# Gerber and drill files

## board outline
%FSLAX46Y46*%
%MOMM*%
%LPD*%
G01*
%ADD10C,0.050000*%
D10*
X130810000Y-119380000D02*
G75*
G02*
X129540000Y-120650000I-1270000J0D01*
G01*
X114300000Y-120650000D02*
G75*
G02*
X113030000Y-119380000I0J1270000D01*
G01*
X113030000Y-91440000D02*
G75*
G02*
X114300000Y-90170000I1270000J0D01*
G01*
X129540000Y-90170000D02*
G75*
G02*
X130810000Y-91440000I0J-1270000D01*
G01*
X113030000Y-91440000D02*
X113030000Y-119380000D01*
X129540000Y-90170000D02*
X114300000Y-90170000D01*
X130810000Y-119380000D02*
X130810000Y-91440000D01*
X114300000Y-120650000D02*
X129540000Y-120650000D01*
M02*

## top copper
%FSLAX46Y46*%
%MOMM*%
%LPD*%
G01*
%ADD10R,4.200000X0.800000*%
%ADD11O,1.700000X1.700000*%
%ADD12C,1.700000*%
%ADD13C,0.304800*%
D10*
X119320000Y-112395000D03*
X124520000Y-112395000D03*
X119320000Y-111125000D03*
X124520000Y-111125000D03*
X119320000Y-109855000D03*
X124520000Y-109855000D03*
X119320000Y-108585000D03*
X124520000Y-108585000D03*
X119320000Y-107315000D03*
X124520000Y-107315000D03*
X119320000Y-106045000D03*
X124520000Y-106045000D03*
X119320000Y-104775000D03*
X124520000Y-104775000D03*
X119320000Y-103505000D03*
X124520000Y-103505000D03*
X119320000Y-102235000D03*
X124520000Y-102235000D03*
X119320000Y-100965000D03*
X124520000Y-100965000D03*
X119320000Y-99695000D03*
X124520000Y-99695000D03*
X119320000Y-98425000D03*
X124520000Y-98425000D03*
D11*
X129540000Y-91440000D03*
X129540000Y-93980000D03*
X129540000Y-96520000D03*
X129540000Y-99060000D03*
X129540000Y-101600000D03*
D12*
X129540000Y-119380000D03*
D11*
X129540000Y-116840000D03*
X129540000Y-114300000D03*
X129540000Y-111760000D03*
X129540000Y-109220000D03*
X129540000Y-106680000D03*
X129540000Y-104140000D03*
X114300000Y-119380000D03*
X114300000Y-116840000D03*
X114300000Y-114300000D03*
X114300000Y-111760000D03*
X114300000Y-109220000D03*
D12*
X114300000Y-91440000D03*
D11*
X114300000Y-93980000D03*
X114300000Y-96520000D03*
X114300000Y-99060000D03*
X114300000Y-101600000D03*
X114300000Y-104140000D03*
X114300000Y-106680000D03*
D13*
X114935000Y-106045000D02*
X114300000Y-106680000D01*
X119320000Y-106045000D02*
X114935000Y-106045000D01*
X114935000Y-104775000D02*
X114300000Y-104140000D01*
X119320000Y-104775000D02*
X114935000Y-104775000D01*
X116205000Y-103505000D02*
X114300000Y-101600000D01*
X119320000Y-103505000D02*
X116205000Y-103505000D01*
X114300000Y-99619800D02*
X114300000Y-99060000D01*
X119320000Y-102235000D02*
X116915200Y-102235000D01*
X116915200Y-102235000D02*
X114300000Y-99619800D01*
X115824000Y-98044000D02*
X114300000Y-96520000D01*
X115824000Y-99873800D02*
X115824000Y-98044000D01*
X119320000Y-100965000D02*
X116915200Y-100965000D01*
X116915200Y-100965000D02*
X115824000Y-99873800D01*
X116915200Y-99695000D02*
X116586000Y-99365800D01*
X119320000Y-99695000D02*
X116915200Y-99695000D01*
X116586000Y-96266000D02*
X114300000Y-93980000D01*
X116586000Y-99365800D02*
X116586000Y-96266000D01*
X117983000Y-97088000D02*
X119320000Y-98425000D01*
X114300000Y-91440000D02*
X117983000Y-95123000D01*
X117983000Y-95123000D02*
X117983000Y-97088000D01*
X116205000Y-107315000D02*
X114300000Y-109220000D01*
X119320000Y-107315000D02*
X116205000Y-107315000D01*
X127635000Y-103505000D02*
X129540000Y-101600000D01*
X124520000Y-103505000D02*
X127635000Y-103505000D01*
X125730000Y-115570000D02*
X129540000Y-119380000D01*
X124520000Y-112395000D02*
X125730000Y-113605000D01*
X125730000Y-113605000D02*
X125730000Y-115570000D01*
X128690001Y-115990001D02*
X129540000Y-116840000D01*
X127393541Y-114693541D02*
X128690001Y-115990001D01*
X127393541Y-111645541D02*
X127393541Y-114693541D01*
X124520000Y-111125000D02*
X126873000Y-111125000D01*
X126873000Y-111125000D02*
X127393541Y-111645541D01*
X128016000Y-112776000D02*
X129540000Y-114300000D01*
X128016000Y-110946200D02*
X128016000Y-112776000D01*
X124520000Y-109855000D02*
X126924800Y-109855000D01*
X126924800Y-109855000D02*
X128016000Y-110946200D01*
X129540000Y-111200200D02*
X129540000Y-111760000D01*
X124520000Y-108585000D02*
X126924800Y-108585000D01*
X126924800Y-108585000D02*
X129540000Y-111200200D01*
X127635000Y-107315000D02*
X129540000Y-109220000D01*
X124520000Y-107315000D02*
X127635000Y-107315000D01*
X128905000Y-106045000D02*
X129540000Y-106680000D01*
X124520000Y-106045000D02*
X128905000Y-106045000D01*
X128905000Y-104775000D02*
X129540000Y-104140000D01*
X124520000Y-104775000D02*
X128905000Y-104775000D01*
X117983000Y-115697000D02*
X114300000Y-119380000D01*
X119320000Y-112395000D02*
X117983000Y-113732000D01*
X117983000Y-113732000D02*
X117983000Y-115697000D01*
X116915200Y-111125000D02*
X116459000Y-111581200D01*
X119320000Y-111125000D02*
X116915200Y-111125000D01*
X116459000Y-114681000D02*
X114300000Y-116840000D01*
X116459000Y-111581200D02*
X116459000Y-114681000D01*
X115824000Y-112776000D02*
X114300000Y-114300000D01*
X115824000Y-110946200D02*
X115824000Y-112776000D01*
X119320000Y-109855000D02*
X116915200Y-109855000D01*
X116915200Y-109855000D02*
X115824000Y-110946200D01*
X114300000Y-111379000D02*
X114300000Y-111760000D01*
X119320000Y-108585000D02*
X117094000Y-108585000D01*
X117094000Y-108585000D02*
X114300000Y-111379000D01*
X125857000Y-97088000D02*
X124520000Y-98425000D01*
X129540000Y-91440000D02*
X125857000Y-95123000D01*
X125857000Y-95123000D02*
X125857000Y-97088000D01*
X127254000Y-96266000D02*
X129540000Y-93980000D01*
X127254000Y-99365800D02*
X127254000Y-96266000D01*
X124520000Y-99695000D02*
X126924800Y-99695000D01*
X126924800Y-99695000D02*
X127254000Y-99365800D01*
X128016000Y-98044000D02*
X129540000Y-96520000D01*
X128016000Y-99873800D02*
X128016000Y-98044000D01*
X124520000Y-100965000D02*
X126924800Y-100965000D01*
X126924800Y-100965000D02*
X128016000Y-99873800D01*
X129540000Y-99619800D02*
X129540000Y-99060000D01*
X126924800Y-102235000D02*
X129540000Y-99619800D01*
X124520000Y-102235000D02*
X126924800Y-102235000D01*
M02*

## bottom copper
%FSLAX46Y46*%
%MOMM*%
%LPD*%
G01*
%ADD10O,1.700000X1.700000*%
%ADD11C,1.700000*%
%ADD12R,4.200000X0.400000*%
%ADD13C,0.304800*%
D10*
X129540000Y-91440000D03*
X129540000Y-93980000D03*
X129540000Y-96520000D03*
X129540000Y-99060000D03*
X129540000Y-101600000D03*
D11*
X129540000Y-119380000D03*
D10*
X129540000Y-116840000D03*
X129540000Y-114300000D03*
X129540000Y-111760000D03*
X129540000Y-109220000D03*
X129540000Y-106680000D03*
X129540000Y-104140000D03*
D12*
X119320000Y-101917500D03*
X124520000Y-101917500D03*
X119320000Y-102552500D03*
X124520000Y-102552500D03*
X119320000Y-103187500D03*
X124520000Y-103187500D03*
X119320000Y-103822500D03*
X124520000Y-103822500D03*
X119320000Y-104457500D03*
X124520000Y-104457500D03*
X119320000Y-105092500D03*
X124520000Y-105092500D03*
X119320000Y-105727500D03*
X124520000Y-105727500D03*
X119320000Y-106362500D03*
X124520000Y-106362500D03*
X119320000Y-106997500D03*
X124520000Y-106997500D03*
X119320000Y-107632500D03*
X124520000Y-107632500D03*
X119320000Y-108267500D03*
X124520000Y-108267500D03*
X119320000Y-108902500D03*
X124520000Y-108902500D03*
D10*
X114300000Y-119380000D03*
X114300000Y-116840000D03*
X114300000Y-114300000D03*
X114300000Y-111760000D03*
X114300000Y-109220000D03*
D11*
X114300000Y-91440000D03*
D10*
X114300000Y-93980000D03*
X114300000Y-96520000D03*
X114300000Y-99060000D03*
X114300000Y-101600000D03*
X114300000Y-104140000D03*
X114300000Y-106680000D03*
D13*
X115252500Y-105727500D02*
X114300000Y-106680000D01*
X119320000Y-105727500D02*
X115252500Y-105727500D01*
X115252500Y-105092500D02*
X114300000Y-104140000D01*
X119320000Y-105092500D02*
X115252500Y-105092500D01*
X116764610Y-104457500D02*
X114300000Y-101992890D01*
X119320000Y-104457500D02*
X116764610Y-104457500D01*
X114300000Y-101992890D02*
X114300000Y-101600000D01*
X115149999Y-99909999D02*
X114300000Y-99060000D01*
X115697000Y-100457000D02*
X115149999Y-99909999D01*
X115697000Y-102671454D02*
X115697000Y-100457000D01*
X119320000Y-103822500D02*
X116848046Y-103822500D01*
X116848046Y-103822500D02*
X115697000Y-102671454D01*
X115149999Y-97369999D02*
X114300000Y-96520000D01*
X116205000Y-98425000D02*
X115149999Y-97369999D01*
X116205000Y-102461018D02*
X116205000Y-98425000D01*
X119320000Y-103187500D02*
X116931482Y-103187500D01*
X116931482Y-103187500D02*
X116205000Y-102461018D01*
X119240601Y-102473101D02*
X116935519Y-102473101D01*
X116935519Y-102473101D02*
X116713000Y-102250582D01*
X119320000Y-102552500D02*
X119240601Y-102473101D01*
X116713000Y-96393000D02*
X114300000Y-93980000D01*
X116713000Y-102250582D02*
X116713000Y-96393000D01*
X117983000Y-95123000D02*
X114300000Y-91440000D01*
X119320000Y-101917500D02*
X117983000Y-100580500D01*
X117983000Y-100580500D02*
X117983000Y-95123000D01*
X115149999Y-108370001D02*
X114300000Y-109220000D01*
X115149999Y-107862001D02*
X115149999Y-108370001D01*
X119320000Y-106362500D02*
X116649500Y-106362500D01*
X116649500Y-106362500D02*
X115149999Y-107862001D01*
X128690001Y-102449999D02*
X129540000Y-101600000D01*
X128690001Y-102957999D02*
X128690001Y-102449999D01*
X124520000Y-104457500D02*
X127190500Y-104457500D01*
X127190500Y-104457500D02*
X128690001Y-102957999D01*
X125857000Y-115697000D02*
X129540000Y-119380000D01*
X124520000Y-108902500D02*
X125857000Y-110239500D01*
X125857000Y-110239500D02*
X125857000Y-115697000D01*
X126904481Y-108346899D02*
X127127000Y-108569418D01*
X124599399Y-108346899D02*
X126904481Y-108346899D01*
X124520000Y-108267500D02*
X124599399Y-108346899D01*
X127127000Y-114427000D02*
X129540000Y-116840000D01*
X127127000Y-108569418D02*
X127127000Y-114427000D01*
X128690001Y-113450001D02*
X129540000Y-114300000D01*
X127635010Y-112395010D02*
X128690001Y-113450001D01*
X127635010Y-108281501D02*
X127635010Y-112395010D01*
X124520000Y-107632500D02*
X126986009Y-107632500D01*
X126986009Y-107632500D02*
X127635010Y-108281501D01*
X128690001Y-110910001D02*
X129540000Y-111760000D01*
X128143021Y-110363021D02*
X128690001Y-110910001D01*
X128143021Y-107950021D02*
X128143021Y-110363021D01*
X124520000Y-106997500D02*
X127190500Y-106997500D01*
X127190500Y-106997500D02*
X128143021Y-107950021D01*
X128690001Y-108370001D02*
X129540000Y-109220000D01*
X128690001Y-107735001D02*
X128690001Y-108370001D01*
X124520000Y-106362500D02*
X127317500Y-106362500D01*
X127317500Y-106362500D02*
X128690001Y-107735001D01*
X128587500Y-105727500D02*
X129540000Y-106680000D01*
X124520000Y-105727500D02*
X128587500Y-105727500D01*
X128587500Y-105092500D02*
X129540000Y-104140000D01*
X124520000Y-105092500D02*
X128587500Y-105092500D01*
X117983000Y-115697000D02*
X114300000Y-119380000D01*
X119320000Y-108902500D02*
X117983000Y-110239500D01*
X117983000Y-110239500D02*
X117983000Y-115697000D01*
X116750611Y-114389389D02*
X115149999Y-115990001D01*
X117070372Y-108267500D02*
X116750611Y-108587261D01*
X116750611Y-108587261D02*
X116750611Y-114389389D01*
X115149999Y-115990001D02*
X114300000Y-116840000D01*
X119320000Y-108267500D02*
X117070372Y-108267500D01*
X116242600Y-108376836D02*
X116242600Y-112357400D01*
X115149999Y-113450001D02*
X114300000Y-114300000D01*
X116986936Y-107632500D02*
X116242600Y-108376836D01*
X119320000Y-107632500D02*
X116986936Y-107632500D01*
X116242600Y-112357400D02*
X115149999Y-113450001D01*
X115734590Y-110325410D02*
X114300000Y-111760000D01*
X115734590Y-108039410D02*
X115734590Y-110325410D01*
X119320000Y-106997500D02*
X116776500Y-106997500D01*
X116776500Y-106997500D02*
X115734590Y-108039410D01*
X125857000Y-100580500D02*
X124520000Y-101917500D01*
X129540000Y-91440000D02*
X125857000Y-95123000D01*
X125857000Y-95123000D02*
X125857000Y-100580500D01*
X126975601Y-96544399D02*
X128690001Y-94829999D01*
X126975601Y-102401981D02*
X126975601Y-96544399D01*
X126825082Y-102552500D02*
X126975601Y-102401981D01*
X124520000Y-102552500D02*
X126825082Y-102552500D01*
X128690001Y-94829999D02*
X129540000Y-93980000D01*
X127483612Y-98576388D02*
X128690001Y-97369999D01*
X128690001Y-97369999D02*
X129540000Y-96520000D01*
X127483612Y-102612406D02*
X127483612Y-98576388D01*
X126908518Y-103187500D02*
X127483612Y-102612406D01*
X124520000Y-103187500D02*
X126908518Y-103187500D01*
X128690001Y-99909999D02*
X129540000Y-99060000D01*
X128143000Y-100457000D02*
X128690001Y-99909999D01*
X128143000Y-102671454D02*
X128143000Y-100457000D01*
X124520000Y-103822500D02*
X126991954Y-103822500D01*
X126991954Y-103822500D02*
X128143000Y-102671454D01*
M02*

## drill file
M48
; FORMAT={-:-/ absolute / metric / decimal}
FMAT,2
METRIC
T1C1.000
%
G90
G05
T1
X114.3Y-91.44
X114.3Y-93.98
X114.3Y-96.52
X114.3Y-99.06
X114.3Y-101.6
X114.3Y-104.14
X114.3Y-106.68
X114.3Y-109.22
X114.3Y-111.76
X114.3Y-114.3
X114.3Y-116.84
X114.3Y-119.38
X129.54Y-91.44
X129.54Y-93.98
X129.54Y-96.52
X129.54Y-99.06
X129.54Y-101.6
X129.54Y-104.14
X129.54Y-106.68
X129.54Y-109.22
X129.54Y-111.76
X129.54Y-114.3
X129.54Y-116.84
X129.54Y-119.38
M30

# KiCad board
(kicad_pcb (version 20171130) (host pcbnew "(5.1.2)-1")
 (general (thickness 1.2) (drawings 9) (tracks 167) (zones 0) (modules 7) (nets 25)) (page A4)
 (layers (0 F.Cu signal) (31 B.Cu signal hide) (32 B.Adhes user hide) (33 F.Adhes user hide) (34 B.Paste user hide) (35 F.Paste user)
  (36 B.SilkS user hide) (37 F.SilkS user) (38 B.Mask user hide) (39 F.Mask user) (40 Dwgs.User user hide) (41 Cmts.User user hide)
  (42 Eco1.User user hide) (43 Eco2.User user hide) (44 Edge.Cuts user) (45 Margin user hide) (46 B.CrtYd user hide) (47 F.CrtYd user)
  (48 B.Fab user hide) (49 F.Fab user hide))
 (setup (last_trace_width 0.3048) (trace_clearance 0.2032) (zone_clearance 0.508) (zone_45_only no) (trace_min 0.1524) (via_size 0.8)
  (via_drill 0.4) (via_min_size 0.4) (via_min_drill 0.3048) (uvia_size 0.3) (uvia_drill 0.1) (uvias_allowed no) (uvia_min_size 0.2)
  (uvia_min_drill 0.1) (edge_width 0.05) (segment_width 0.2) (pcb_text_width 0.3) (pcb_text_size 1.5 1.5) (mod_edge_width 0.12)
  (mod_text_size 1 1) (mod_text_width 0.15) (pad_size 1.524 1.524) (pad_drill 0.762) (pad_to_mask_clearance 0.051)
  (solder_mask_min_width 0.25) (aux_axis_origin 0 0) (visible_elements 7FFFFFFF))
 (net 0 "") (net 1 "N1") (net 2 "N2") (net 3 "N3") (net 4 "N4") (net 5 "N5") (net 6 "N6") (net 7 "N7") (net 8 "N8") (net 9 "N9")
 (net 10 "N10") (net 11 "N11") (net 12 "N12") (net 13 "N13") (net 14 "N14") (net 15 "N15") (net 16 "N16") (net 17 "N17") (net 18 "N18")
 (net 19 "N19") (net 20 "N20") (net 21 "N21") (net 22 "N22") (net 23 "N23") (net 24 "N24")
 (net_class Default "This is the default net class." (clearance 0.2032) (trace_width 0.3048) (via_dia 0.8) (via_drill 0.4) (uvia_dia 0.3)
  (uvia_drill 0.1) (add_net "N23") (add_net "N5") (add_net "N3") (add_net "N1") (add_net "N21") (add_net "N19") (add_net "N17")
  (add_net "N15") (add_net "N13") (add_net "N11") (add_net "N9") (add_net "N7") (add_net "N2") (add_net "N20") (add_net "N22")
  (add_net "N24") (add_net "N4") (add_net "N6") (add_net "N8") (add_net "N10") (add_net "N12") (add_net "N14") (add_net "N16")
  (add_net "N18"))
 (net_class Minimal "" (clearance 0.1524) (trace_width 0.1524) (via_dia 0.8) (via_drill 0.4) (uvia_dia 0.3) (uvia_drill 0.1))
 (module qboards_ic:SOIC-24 (layer F.Cu) (at 121.92 105.41 270)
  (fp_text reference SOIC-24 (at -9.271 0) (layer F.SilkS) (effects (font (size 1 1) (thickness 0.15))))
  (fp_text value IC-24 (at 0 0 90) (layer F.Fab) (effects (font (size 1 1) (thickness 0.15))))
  (pad 12 smd rect (at 6.985 2.6 270) (size 0.8 4.2) (layers F.Cu F.Paste F.Mask) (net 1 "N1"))
  (pad 13 smd rect (at 6.985 -2.6 270) (size 0.8 4.2) (layers F.Cu F.Paste F.Mask) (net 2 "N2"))
  (pad 11 smd rect (at 5.715 2.6 270) (size 0.8 4.2) (layers F.Cu F.Paste F.Mask) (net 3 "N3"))
  (pad 14 smd rect (at 5.715 -2.6 270) (size 0.8 4.2) (layers F.Cu F.Paste F.Mask) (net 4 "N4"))
  (pad 10 smd rect (at 4.445 2.6 270) (size 0.8 4.2) (layers F.Cu F.Paste F.Mask) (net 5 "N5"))
  (pad 15 smd rect (at 4.445 -2.6 270) (size 0.8 4.2) (layers F.Cu F.Paste F.Mask) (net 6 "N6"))
  (pad 9 smd rect (at 3.175 2.6 270) (size 0.8 4.2) (layers F.Cu F.Paste F.Mask) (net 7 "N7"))
  (pad 16 smd rect (at 3.175 -2.6 270) (size 0.8 4.2) (layers F.Cu F.Paste F.Mask) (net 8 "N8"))
  (pad 8 smd rect (at 1.905 2.6 270) (size 0.8 4.2) (layers F.Cu F.Paste F.Mask) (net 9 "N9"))
  (pad 17 smd rect (at 1.905 -2.6 270) (size 0.8 4.2) (layers F.Cu F.Paste F.Mask) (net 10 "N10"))
  (pad 7 smd rect (at 0.635 2.6 270) (size 0.8 4.2) (layers F.Cu F.Paste F.Mask) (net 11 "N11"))
  (pad 18 smd rect (at 0.635 -2.6 270) (size 0.8 4.2) (layers F.Cu F.Paste F.Mask) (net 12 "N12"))
  (pad 6 smd rect (at -0.635 2.6 270) (size 0.8 4.2) (layers F.Cu F.Paste F.Mask) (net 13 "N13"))
  (pad 19 smd rect (at -0.635 -2.6 270) (size 0.8 4.2) (layers F.Cu F.Paste F.Mask) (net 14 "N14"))
  (pad 5 smd rect (at -1.905 2.6 270) (size 0.8 4.2) (layers F.Cu F.Paste F.Mask) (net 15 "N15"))
  (pad 20 smd rect (at -1.905 -2.6 270) (size 0.8 4.2) (layers F.Cu F.Paste F.Mask) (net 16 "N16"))
  (pad 4 smd rect (at -3.175 2.6 270) (size 0.8 4.2) (layers F.Cu F.Paste F.Mask) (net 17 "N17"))
  (pad 21 smd rect (at -3.175 -2.6 270) (size 0.8 4.2) (layers F.Cu F.Paste F.Mask) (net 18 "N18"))
  (pad 3 smd rect (at -4.445 2.6 270) (size 0.8 4.2) (layers F.Cu F.Paste F.Mask) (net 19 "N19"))
  (pad 22 smd rect (at -4.445 -2.6 270) (size 0.8 4.2) (layers F.Cu F.Paste F.Mask) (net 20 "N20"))
  (pad 2 smd rect (at -5.715 2.6 270) (size 0.8 4.2) (layers F.Cu F.Paste F.Mask) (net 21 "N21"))
  (pad 23 smd rect (at -5.715 -2.6 270) (size 0.8 4.2) (layers F.Cu F.Paste F.Mask) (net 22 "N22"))
  (pad 1 smd rect (at -6.985 2.6 270) (size 0.8 4.2) (layers F.Cu F.Paste F.Mask) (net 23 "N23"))
  (pad 24 smd rect (at -6.985 -2.6 270) (size 0.8 4.2) (layers F.Cu F.Paste F.Mask) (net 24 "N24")))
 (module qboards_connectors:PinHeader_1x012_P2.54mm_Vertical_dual (layer F.Cu) (at 129.54 119.38 180)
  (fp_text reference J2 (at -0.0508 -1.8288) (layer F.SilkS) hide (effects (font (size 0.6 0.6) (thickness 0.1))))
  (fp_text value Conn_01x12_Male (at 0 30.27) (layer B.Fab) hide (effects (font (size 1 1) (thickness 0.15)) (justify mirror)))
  (pad 12 thru_hole oval (at 0 27.94 180) (size 1.7 1.7) (drill 1) (layers *.Cu *.Mask) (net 24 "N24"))
  (pad 11 thru_hole oval (at 0 25.4 180) (size 1.7 1.7) (drill 1) (layers *.Cu *.Mask) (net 22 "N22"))
  (pad 10 thru_hole oval (at 0 22.86 180) (size 1.7 1.7) (drill 1) (layers *.Cu *.Mask) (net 20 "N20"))
  (pad 9 thru_hole oval (at 0 20.32 180) (size 1.7 1.7) (drill 1) (layers *.Cu *.Mask) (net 18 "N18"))
  (pad 8 thru_hole oval (at 0 17.78 180) (size 1.7 1.7) (drill 1) (layers *.Cu *.Mask) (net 16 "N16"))
  (pad 1 thru_hole circle (at 0 0 180) (size 1.7 1.7) (drill 1) (layers *.Cu *.Mask) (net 2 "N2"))
  (pad 2 thru_hole oval (at 0 2.54 180) (size 1.7 1.7) (drill 1) (layers *.Cu *.Mask) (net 4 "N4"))
  (pad 3 thru_hole oval (at 0 5.08 180) (size 1.7 1.7) (drill 1) (layers *.Cu *.Mask) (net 6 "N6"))
  (pad 4 thru_hole oval (at 0 7.62 180) (size 1.7 1.7) (drill 1) (layers *.Cu *.Mask) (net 8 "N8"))
  (pad 5 thru_hole oval (at 0 10.16 180) (size 1.7 1.7) (drill 1) (layers *.Cu *.Mask) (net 10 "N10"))
  (pad 6 thru_hole oval (at 0 12.7 180) (size 1.7 1.7) (drill 1) (layers *.Cu *.Mask) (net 12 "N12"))
  (pad 7 thru_hole oval (at 0 15.24 180) (size 1.7 1.7) (drill 1) (layers *.Cu *.Mask) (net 14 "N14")))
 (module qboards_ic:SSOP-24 (layer B.Cu) (at 121.92 105.41 90)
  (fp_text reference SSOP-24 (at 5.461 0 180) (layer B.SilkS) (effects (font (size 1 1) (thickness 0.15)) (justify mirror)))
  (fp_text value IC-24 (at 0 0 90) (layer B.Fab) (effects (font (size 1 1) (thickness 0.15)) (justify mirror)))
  (pad 12 smd rect (at 3.4925 -2.6 90) (size 0.4 4.2) (layers B.Cu B.Paste B.Mask) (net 23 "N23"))
  (pad 13 smd rect (at 3.4925 2.6 90) (size 0.4 4.2) (layers B.Cu B.Paste B.Mask) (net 24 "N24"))
  (pad 11 smd rect (at 2.8575 -2.6 90) (size 0.4 4.2) (layers B.Cu B.Paste B.Mask) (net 21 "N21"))
  (pad 14 smd rect (at 2.8575 2.6 90) (size 0.4 4.2) (layers B.Cu B.Paste B.Mask) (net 22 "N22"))
  (pad 10 smd rect (at 2.2225 -2.6 90) (size 0.4 4.2) (layers B.Cu B.Paste B.Mask) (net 19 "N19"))
  (pad 15 smd rect (at 2.2225 2.6 90) (size 0.4 4.2) (layers B.Cu B.Paste B.Mask) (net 20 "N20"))
  (pad 9 smd rect (at 1.5875 -2.6 90) (size 0.4 4.2) (layers B.Cu B.Paste B.Mask) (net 17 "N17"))
  (pad 16 smd rect (at 1.5875 2.6 90) (size 0.4 4.2) (layers B.Cu B.Paste B.Mask) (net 18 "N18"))
  (pad 8 smd rect (at 0.9525 -2.6 90) (size 0.4 4.2) (layers B.Cu B.Paste B.Mask) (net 15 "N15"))
  (pad 17 smd rect (at 0.9525 2.6 90) (size 0.4 4.2) (layers B.Cu B.Paste B.Mask) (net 16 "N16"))
  (pad 7 smd rect (at 0.3175 -2.6 90) (size 0.4 4.2) (layers B.Cu B.Paste B.Mask) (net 13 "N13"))
  (pad 18 smd rect (at 0.3175 2.6 90) (size 0.4 4.2) (layers B.Cu B.Paste B.Mask) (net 14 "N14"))
  (pad 6 smd rect (at -0.3175 -2.6 90) (size 0.4 4.2) (layers B.Cu B.Paste B.Mask) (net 11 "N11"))
  (pad 19 smd rect (at -0.3175 2.6 90) (size 0.4 4.2) (layers B.Cu B.Paste B.Mask) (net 12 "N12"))
  (pad 5 smd rect (at -0.9525 -2.6 90) (size 0.4 4.2) (layers B.Cu B.Paste B.Mask) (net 9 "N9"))
  (pad 20 smd rect (at -0.9525 2.6 90) (size 0.4 4.2) (layers B.Cu B.Paste B.Mask) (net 10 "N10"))
  (pad 4 smd rect (at -1.5875 -2.6 90) (size 0.4 4.2) (layers B.Cu B.Paste B.Mask) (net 7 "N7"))
  (pad 21 smd rect (at -1.5875 2.6 90) (size 0.4 4.2) (layers B.Cu B.Paste B.Mask) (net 8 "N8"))
  (pad 3 smd rect (at -2.2225 -2.6 90) (size 0.4 4.2) (layers B.Cu B.Paste B.Mask) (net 5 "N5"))
  (pad 22 smd rect (at -2.2225 2.6 90) (size 0.4 4.2) (layers B.Cu B.Paste B.Mask) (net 6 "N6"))
  (pad 2 smd rect (at -2.8575 -2.6 90) (size 0.4 4.2) (layers B.Cu B.Paste B.Mask) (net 3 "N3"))
  (pad 23 smd rect (at -2.8575 2.6 90) (size 0.4 4.2) (layers B.Cu B.Paste B.Mask) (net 4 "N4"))
  (pad 1 smd rect (at -3.4925 -2.6 90) (size 0.4 4.2) (layers B.Cu B.Paste B.Mask) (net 1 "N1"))
  (pad 24 smd rect (at -3.4925 2.6 90) (size 0.4 4.2) (layers B.Cu B.Paste B.Mask) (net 2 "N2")))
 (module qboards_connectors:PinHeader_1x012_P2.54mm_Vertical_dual (layer F.Cu) (at 114.3 91.44)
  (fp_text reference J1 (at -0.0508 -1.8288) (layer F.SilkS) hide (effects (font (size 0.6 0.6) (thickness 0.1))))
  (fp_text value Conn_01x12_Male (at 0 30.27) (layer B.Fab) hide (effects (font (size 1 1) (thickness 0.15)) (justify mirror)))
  (pad 12 thru_hole oval (at 0 27.94) (size 1.7 1.7) (drill 1) (layers *.Cu *.Mask) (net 1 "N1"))
  (pad 11 thru_hole oval (at 0 25.4) (size 1.7 1.7) (drill 1) (layers *.Cu *.Mask) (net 3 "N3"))
  (pad 10 thru_hole oval (at 0 22.86) (size 1.7 1.7) (drill 1) (layers *.Cu *.Mask) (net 5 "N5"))
  (pad 9 thru_hole oval (at 0 20.32) (size 1.7 1.7) (drill 1) (layers *.Cu *.Mask) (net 7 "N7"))
  (pad 8 thru_hole oval (at 0 17.78) (size 1.7 1.7) (drill 1) (layers *.Cu *.Mask) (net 9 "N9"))
  (pad 1 thru_hole circle (at 0 0) (size 1.7 1.7) (drill 1) (layers *.Cu *.Mask) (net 23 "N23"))
  (pad 2 thru_hole oval (at 0 2.54) (size 1.7 1.7) (drill 1) (layers *.Cu *.Mask) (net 21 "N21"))
  (pad 3 thru_hole oval (at 0 5.08) (size 1.7 1.7) (drill 1) (layers *.Cu *.Mask) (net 19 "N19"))
  (pad 4 thru_hole oval (at 0 7.62) (size 1.7 1.7) (drill 1) (layers *.Cu *.Mask) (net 17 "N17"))
  (pad 5 thru_hole oval (at 0 10.16) (size 1.7 1.7) (drill 1) (layers *.Cu *.Mask) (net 15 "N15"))
  (pad 6 thru_hole oval (at 0 12.7) (size 1.7 1.7) (drill 1) (layers *.Cu *.Mask) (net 13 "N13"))
  (pad 7 thru_hole oval (at 0 15.24) (size 1.7 1.7) (drill 1) (layers *.Cu *.Mask) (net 11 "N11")))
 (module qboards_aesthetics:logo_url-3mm (layer F.Cu) (at 117.602 117.983)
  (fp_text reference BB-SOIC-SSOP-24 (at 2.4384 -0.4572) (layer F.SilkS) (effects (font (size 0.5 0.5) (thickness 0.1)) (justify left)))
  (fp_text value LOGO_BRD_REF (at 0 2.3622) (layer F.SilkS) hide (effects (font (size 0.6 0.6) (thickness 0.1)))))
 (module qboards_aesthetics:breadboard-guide (layer F.Cu) (at 99.06 91.44)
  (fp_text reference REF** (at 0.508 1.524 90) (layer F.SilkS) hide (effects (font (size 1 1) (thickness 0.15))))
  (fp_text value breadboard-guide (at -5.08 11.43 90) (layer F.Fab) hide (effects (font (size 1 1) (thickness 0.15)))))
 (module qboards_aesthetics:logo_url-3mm (layer B.Cu) (at 126.492 117.983 180)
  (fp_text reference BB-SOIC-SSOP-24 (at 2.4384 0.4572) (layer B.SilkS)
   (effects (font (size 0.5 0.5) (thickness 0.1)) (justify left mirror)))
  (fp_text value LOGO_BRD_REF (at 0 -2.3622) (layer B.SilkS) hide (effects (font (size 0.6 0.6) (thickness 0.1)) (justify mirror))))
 (gr_arc (start 129.54 119.38) (end 129.54 120.65) (angle -90) (layer Edge.Cuts) (width 0.05))
 (gr_arc (start 114.3 119.38) (end 113.03 119.38) (angle -90) (layer Edge.Cuts) (width 0.05))
 (gr_arc (start 114.3 91.44) (end 114.3 90.17) (angle -90) (layer Edge.Cuts) (width 0.05))
 (gr_arc (start 129.54 91.44) (end 130.81 91.44) (angle -90) (layer Edge.Cuts) (width 0.05))
 (gr_line (start 113.03 91.44) (end 113.03 119.38) (layer Edge.Cuts) (width 0.05))
 (gr_line (start 129.54 90.17) (end 114.3 90.17) (layer Edge.Cuts) (width 0.05))
 (gr_line (start 130.81 119.38) (end 130.81 91.44) (layer Edge.Cuts) (width 0.05))
 (gr_line (start 114.3 120.65) (end 129.54 120.65) (layer Edge.Cuts) (width 0.05))
 (segment (start 114.935 106.045) (end 114.3 106.68) (width 0.3048) (layer F.Cu) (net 11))
 (segment (start 119.32 106.045) (end 114.935 106.045) (width 0.3048) (layer F.Cu) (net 11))
 (segment (start 115.2525 105.7275) (end 114.3 106.68) (width 0.3048) (layer B.Cu) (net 11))
 (segment (start 119.32 105.7275) (end 115.2525 105.7275) (width 0.3048) (layer B.Cu) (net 11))
 (segment (start 114.935 104.775) (end 114.3 104.14) (width 0.3048) (layer F.Cu) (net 13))
 (segment (start 119.32 104.775) (end 114.935 104.775) (width 0.3048) (layer F.Cu) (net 13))
 (segment (start 115.2525 105.0925) (end 114.3 104.14) (width 0.3048) (layer B.Cu) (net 13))
 (segment (start 119.32 105.0925) (end 115.2525 105.0925) (width 0.3048) (layer B.Cu) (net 13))
 (segment (start 116.205 103.505) (end 114.3 101.6) (width 0.3048) (layer F.Cu) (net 15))
 (segment (start 119.32 103.505) (end 116.205 103.505) (width 0.3048) (layer F.Cu) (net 15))
 (segment (start 116.76461 104.4575) (end 114.3 101.99289) (width 0.3048) (layer B.Cu) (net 15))
 (segment (start 119.32 104.4575) (end 116.76461 104.4575) (width 0.3048) (layer B.Cu) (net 15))
 (segment (start 114.3 101.99289) (end 114.3 101.6) (width 0.3048) (layer B.Cu) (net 15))
 (segment (start 114.3 99.6198) (end 114.3 99.06) (width 0.3048) (layer F.Cu) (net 17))
 (segment (start 119.32 102.235) (end 116.9152 102.235) (width 0.3048) (layer F.Cu) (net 17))
 (segment (start 116.9152 102.235) (end 114.3 99.6198) (width 0.3048) (layer F.Cu) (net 17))
 (segment (start 115.149999 99.909999) (end 114.3 99.06) (width 0.3048) (layer B.Cu) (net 17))
 (segment (start 115.697 100.457) (end 115.149999 99.909999) (width 0.3048) (layer B.Cu) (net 17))
 (segment (start 115.697 102.671454) (end 115.697 100.457) (width 0.3048) (layer B.Cu) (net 17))
 (segment (start 119.32 103.8225) (end 116.848046 103.8225) (width 0.3048) (layer B.Cu) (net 17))
 (segment (start 116.848046 103.8225) (end 115.697 102.671454) (width 0.3048) (layer B.Cu) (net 17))
 (segment (start 115.824 98.044) (end 114.3 96.52) (width 0.3048) (layer F.Cu) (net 19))
 (segment (start 115.824 99.8738) (end 115.824 98.044) (width 0.3048) (layer F.Cu) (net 19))
 (segment (start 119.32 100.965) (end 116.9152 100.965) (width 0.3048) (layer F.Cu) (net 19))
 (segment (start 116.9152 100.965) (end 115.824 99.8738) (width 0.3048) (layer F.Cu) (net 19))
 (segment (start 115.149999 97.369999) (end 114.3 96.52) (width 0.3048) (layer B.Cu) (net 19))
 (segment (start 116.205 98.425) (end 115.149999 97.369999) (width 0.3048) (layer B.Cu) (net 19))
 (segment (start 116.205 102.461018) (end 116.205 98.425) (width 0.3048) (layer B.Cu) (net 19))
 (segment (start 119.32 103.1875) (end 116.931482 103.1875) (width 0.3048) (layer B.Cu) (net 19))
 (segment (start 116.931482 103.1875) (end 116.205 102.461018) (width 0.3048) (layer B.Cu) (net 19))
 (segment (start 116.9152 99.695) (end 116.586 99.3658) (width 0.3048) (layer F.Cu) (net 21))
 (segment (start 119.32 99.695) (end 116.9152 99.695) (width 0.3048) (layer F.Cu) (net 21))
 (segment (start 116.586 96.266) (end 114.3 93.98) (width 0.3048) (layer F.Cu) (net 21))
 (segment (start 116.586 99.3658) (end 116.586 96.266) (width 0.3048) (layer F.Cu) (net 21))
 (segment (start 119.240601 102.473101) (end 116.935519 102.473101) (width 0.3048) (layer B.Cu) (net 21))
 (segment (start 116.935519 102.473101) (end 116.713 102.250582) (width 0.3048) (layer B.Cu) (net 21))
 (segment (start 119.32 102.5525) (end 119.240601 102.473101) (width 0.3048) (layer B.Cu) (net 21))
 (segment (start 116.713 96.393) (end 114.3 93.98) (width 0.3048) (layer B.Cu) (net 21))
 (segment (start 116.713 102.250582) (end 116.713 96.393) (width 0.3048) (layer B.Cu) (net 21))
 (segment (start 117.983 95.123) (end 114.3 91.44) (width 0.3048) (layer B.Cu) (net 23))
 (segment (start 119.32 101.9175) (end 117.983 100.5805) (width 0.3048) (layer B.Cu) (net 23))
 (segment (start 117.983 100.5805) (end 117.983 95.123) (width 0.3048) (layer B.Cu) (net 23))
 (segment (start 117.983 97.088) (end 119.32 98.425) (width 0.3048) (layer F.Cu) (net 23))
 (segment (start 114.3 91.44) (end 117.983 95.123) (width 0.3048) (layer F.Cu) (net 23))
 (segment (start 117.983 95.123) (end 117.983 97.088) (width 0.3048) (layer F.Cu) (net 23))
 (segment (start 116.205 107.315) (end 114.3 109.22) (width 0.3048) (layer F.Cu) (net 9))
 (segment (start 119.32 107.315) (end 116.205 107.315) (width 0.3048) (layer F.Cu) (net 9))
 (segment (start 115.149999 108.370001) (end 114.3 109.22) (width 0.3048) (layer B.Cu) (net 9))
 (segment (start 115.149999 107.862001) (end 115.149999 108.370001) (width 0.3048) (layer B.Cu) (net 9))
 (segment (start 119.32 106.3625) (end 116.6495 106.3625) (width 0.3048) (layer B.Cu) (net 9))
 (segment (start 116.6495 106.3625) (end 115.149999 107.862001) (width 0.3048) (layer B.Cu) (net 9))
 (segment (start 127.635 103.505) (end 129.54 101.6) (width 0.3048) (layer F.Cu) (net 16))
 (segment (start 124.52 103.505) (end 127.635 103.505) (width 0.3048) (layer F.Cu) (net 16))
 (segment (start 128.690001 102.449999) (end 129.54 101.6) (width 0.3048) (layer B.Cu) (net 16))
 (segment (start 128.690001 102.957999) (end 128.690001 102.449999) (width 0.3048) (layer B.Cu) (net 16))
 (segment (start 124.52 104.4575) (end 127.1905 104.4575) (width 0.3048) (layer B.Cu) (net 16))
 (segment (start 127.1905 104.4575) (end 128.690001 102.957999) (width 0.3048) (layer B.Cu) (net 16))
 (segment (start 125.857 115.697) (end 129.54 119.38) (width 0.3048) (layer B.Cu) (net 2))
 (segment (start 124.52 108.9025) (end 125.857 110.2395) (width 0.3048) (layer B.Cu) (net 2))
 (segment (start 125.857 110.2395) (end 125.857 115.697) (width 0.3048) (layer B.Cu) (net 2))
 (segment (start 125.73 115.57) (end 129.54 119.38) (width 0.3048) (layer F.Cu) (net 2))
 (segment (start 124.52 112.395) (end 125.73 113.605) (width 0.3048) (layer F.Cu) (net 2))
 (segment (start 125.73 113.605) (end 125.73 115.57) (width 0.3048) (layer F.Cu) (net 2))
 (segment (start 128.690001 115.990001) (end 129.54 116.84) (width 0.3048) (layer F.Cu) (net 4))
 (segment (start 127.393541 114.693541) (end 128.690001 115.990001) (width 0.3048) (layer F.Cu) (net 4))
 (segment (start 127.393541 111.645541) (end 127.393541 114.693541) (width 0.3048) (layer F.Cu) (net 4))
 (segment (start 124.52 111.125) (end 126.873 111.125) (width 0.3048) (layer F.Cu) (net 4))
 (segment (start 126.873 111.125) (end 127.393541 111.645541) (width 0.3048) (layer F.Cu) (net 4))
 (segment (start 126.904481 108.346899) (end 127.127 108.569418) (width 0.3048) (layer B.Cu) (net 4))
 (segment (start 124.599399 108.346899) (end 126.904481 108.346899) (width 0.3048) (layer B.Cu) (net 4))
 (segment (start 124.52 108.2675) (end 124.599399 108.346899) (width 0.3048) (layer B.Cu) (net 4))
 (segment (start 127.127 114.427) (end 129.54 116.84) (width 0.3048) (layer B.Cu) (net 4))
 (segment (start 127.127 108.569418) (end 127.127 114.427) (width 0.3048) (layer B.Cu) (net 4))
 (segment (start 128.016 112.776) (end 129.54 114.3) (width 0.3048) (layer F.Cu) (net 6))
 (segment (start 128.016 110.9462) (end 128.016 112.776) (width 0.3048) (layer F.Cu) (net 6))
 (segment (start 124.52 109.855) (end 126.9248 109.855) (width 0.3048) (layer F.Cu) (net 6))
 (segment (start 126.9248 109.855) (end 128.016 110.9462) (width 0.3048) (layer F.Cu) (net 6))
 (segment (start 128.690001 113.450001) (end 129.54 114.3) (width 0.3048) (layer B.Cu) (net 6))
 (segment (start 127.63501 112.39501) (end 128.690001 113.450001) (width 0.3048) (layer B.Cu) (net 6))
 (segment (start 127.63501 108.281501) (end 127.63501 112.39501) (width 0.3048) (layer B.Cu) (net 6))
 (segment (start 124.52 107.6325) (end 126.986009 107.6325) (width 0.3048) (layer B.Cu) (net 6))
 (segment (start 126.986009 107.6325) (end 127.63501 108.281501) (width 0.3048) (layer B.Cu) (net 6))
 (segment (start 129.54 111.2002) (end 129.54 111.76) (width 0.3048) (layer F.Cu) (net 8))
 (segment (start 124.52 108.585) (end 126.9248 108.585) (width 0.3048) (layer F.Cu) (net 8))
 (segment (start 126.9248 108.585) (end 129.54 111.2002) (width 0.3048) (layer F.Cu) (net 8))
 (segment (start 128.690001 110.910001) (end 129.54 111.76) (width 0.3048) (layer B.Cu) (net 8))
 (segment (start 128.143021 110.363021) (end 128.690001 110.910001) (width 0.3048) (layer B.Cu) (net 8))
 (segment (start 128.143021 107.950021) (end 128.143021 110.363021) (width 0.3048) (layer B.Cu) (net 8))
 (segment (start 124.52 106.9975) (end 127.1905 106.9975) (width 0.3048) (layer B.Cu) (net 8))
 (segment (start 127.1905 106.9975) (end 128.143021 107.950021) (width 0.3048) (layer B.Cu) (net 8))
 (segment (start 127.635 107.315) (end 129.54 109.22) (width 0.3048) (layer F.Cu) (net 10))
 (segment (start 124.52 107.315) (end 127.635 107.315) (width 0.3048) (layer F.Cu) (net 10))
 (segment (start 128.690001 108.370001) (end 129.54 109.22) (width 0.3048) (layer B.Cu) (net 10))
 (segment (start 128.690001 107.735001) (end 128.690001 108.370001) (width 0.3048) (layer B.Cu) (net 10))
 (segment (start 124.52 106.3625) (end 127.3175 106.3625) (width 0.3048) (layer B.Cu) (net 10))
 (segment (start 127.3175 106.3625) (end 128.690001 107.735001) (width 0.3048) (layer B.Cu) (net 10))
 (segment (start 128.905 106.045) (end 129.54 106.68) (width 0.3048) (layer F.Cu) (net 12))
 (segment (start 124.52 106.045) (end 128.905 106.045) (width 0.3048) (layer F.Cu) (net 12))
 (segment (start 128.5875 105.7275) (end 129.54 106.68) (width 0.3048) (layer B.Cu) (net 12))
 (segment (start 124.52 105.7275) (end 128.5875 105.7275) (width 0.3048) (layer B.Cu) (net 12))
 (segment (start 128.905 104.775) (end 129.54 104.14) (width 0.3048) (layer F.Cu) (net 14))
 (segment (start 124.52 104.775) (end 128.905 104.775) (width 0.3048) (layer F.Cu) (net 14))
 (segment (start 128.5875 105.0925) (end 129.54 104.14) (width 0.3048) (layer B.Cu) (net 14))
 (segment (start 124.52 105.0925) (end 128.5875 105.0925) (width 0.3048) (layer B.Cu) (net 14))
 (segment (start 117.983 115.697) (end 114.3 119.38) (width 0.3048) (layer B.Cu) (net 1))
 (segment (start 119.32 108.9025) (end 117.983 110.2395) (width 0.3048) (layer B.Cu) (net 1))
 (segment (start 117.983 110.2395) (end 117.983 115.697) (width 0.3048) (layer B.Cu) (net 1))
 (segment (start 117.983 115.697) (end 114.3 119.38) (width 0.3048) (layer F.Cu) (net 1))
 (segment (start 119.32 112.395) (end 117.983 113.732) (width 0.3048) (layer F.Cu) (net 1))
 (segment (start 117.983 113.732) (end 117.983 115.697) (width 0.3048) (layer F.Cu) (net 1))
 (segment (start 116.9152 111.125) (end 116.459 111.5812) (width 0.3048) (layer F.Cu) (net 3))
 (segment (start 119.32 111.125) (end 116.9152 111.125) (width 0.3048) (layer F.Cu) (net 3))
 (segment (start 116.459 114.681) (end 114.3 116.84) (width 0.3048) (layer F.Cu) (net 3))
 (segment (start 116.459 111.5812) (end 116.459 114.681) (width 0.3048) (layer F.Cu) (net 3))
 (segment (start 116.750611 114.389389) (end 115.149999 115.990001) (width 0.3048) (layer B.Cu) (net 3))
 (segment (start 117.070372 108.2675) (end 116.750611 108.587261) (width 0.3048) (layer B.Cu) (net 3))
 (segment (start 116.750611 108.587261) (end 116.750611 114.389389) (width 0.3048) (layer B.Cu) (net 3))
 (segment (start 115.149999 115.990001) (end 114.3 116.84) (width 0.3048) (layer B.Cu) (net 3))
 (segment (start 119.32 108.2675) (end 117.070372 108.2675) (width 0.3048) (layer B.Cu) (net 3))
 (segment (start 115.824 112.776) (end 114.3 114.3) (width 0.3048) (layer F.Cu) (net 5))
 (segment (start 115.824 110.9462) (end 115.824 112.776) (width 0.3048) (layer F.Cu) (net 5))
 (segment (start 119.32 109.855) (end 116.9152 109.855) (width 0.3048) (layer F.Cu) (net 5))
 (segment (start 116.9152 109.855) (end 115.824 110.9462) (width 0.3048) (layer F.Cu) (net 5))
 (segment (start 116.2426 108.376836) (end 116.2426 112.3574) (width 0.3048) (layer B.Cu) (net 5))
 (segment (start 115.149999 113.450001) (end 114.3 114.3) (width 0.3048) (layer B.Cu) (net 5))
 (segment (start 116.986936 107.6325) (end 116.2426 108.376836) (width 0.3048) (layer B.Cu) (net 5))
 (segment (start 119.32 107.6325) (end 116.986936 107.6325) (width 0.3048) (layer B.Cu) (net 5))
 (segment (start 116.2426 112.3574) (end 115.149999 113.450001) (width 0.3048) (layer B.Cu) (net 5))
 (segment (start 114.3 111.379) (end 114.3 111.76) (width 0.3048) (layer F.Cu) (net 7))
 (segment (start 119.32 108.585) (end 117.094 108.585) (width 0.3048) (layer F.Cu) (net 7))
 (segment (start 117.094 108.585) (end 114.3 111.379) (width 0.3048) (layer F.Cu) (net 7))
 (segment (start 115.73459 110.32541) (end 114.3 111.76) (width 0.3048) (layer B.Cu) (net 7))
 (segment (start 115.73459 108.03941) (end 115.73459 110.32541) (width 0.3048) (layer B.Cu) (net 7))
 (segment (start 119.32 106.9975) (end 116.7765 106.9975) (width 0.3048) (layer B.Cu) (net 7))
 (segment (start 116.7765 106.9975) (end 115.73459 108.03941) (width 0.3048) (layer B.Cu) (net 7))
 (segment (start 125.857 100.5805) (end 124.52 101.9175) (width 0.3048) (layer B.Cu) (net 24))
 (segment (start 129.54 91.44) (end 125.857 95.123) (width 0.3048) (layer B.Cu) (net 24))
 (segment (start 125.857 95.123) (end 125.857 100.5805) (width 0.3048) (layer B.Cu) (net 24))
 (segment (start 125.857 97.088) (end 124.52 98.425) (width 0.3048) (layer F.Cu) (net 24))
 (segment (start 129.54 91.44) (end 125.857 95.123) (width 0.3048) (layer F.Cu) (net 24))
 (segment (start 125.857 95.123) (end 125.857 97.088) (width 0.3048) (layer F.Cu) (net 24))
 (segment (start 127.254 96.266) (end 129.54 93.98) (width 0.3048) (layer F.Cu) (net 22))
 (segment (start 127.254 99.3658) (end 127.254 96.266) (width 0.3048) (layer F.Cu) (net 22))
 (segment (start 124.52 99.695) (end 126.9248 99.695) (width 0.3048) (layer F.Cu) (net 22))
 (segment (start 126.9248 99.695) (end 127.254 99.3658) (width 0.3048) (layer F.Cu) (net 22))
 (segment (start 126.975601 96.544399) (end 128.690001 94.829999) (width 0.3048) (layer B.Cu) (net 22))
 (segment (start 126.975601 102.401981) (end 126.975601 96.544399) (width 0.3048) (layer B.Cu) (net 22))
 (segment (start 126.825082 102.5525) (end 126.975601 102.401981) (width 0.3048) (layer B.Cu) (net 22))
 (segment (start 124.52 102.5525) (end 126.825082 102.5525) (width 0.3048) (layer B.Cu) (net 22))
 (segment (start 128.690001 94.829999) (end 129.54 93.98) (width 0.3048) (layer B.Cu) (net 22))
 (segment (start 128.016 98.044) (end 129.54 96.52) (width 0.3048) (layer F.Cu) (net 20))
 (segment (start 128.016 99.8738) (end 128.016 98.044) (width 0.3048) (layer F.Cu) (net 20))
 (segment (start 124.52 100.965) (end 126.9248 100.965) (width 0.3048) (layer F.Cu) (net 20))
 (segment (start 126.9248 100.965) (end 128.016 99.8738) (width 0.3048) (layer F.Cu) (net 20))
 (segment (start 127.483612 98.576388) (end 128.690001 97.369999) (width 0.3048) (layer B.Cu) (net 20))
 (segment (start 128.690001 97.369999) (end 129.54 96.52) (width 0.3048) (layer B.Cu) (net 20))
 (segment (start 127.483612 102.612406) (end 127.483612 98.576388) (width 0.3048) (layer B.Cu) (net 20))
 (segment (start 126.908518 103.1875) (end 127.483612 102.612406) (width 0.3048) (layer B.Cu) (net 20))
 (segment (start 124.52 103.1875) (end 126.908518 103.1875) (width 0.3048) (layer B.Cu) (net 20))
 (segment (start 129.54 99.6198) (end 129.54 99.06) (width 0.3048) (layer F.Cu) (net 18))
 (segment (start 126.9248 102.235) (end 129.54 99.6198) (width 0.3048) (layer F.Cu) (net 18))
 (segment (start 124.52 102.235) (end 126.9248 102.235) (width 0.3048) (layer F.Cu) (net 18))
 (segment (start 128.690001 99.909999) (end 129.54 99.06) (width 0.3048) (layer B.Cu) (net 18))
 (segment (start 128.143 100.457) (end 128.690001 99.909999) (width 0.3048) (layer B.Cu) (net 18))
 (segment (start 128.143 102.671454) (end 128.143 100.457) (width 0.3048) (layer B.Cu) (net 18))
 (segment (start 124.52 103.8225) (end 126.991954 103.8225) (width 0.3048) (layer B.Cu) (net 18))
 (segment (start 126.991954 103.8225) (end 128.143 102.671454) (width 0.3048) (layer B.Cu) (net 18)))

